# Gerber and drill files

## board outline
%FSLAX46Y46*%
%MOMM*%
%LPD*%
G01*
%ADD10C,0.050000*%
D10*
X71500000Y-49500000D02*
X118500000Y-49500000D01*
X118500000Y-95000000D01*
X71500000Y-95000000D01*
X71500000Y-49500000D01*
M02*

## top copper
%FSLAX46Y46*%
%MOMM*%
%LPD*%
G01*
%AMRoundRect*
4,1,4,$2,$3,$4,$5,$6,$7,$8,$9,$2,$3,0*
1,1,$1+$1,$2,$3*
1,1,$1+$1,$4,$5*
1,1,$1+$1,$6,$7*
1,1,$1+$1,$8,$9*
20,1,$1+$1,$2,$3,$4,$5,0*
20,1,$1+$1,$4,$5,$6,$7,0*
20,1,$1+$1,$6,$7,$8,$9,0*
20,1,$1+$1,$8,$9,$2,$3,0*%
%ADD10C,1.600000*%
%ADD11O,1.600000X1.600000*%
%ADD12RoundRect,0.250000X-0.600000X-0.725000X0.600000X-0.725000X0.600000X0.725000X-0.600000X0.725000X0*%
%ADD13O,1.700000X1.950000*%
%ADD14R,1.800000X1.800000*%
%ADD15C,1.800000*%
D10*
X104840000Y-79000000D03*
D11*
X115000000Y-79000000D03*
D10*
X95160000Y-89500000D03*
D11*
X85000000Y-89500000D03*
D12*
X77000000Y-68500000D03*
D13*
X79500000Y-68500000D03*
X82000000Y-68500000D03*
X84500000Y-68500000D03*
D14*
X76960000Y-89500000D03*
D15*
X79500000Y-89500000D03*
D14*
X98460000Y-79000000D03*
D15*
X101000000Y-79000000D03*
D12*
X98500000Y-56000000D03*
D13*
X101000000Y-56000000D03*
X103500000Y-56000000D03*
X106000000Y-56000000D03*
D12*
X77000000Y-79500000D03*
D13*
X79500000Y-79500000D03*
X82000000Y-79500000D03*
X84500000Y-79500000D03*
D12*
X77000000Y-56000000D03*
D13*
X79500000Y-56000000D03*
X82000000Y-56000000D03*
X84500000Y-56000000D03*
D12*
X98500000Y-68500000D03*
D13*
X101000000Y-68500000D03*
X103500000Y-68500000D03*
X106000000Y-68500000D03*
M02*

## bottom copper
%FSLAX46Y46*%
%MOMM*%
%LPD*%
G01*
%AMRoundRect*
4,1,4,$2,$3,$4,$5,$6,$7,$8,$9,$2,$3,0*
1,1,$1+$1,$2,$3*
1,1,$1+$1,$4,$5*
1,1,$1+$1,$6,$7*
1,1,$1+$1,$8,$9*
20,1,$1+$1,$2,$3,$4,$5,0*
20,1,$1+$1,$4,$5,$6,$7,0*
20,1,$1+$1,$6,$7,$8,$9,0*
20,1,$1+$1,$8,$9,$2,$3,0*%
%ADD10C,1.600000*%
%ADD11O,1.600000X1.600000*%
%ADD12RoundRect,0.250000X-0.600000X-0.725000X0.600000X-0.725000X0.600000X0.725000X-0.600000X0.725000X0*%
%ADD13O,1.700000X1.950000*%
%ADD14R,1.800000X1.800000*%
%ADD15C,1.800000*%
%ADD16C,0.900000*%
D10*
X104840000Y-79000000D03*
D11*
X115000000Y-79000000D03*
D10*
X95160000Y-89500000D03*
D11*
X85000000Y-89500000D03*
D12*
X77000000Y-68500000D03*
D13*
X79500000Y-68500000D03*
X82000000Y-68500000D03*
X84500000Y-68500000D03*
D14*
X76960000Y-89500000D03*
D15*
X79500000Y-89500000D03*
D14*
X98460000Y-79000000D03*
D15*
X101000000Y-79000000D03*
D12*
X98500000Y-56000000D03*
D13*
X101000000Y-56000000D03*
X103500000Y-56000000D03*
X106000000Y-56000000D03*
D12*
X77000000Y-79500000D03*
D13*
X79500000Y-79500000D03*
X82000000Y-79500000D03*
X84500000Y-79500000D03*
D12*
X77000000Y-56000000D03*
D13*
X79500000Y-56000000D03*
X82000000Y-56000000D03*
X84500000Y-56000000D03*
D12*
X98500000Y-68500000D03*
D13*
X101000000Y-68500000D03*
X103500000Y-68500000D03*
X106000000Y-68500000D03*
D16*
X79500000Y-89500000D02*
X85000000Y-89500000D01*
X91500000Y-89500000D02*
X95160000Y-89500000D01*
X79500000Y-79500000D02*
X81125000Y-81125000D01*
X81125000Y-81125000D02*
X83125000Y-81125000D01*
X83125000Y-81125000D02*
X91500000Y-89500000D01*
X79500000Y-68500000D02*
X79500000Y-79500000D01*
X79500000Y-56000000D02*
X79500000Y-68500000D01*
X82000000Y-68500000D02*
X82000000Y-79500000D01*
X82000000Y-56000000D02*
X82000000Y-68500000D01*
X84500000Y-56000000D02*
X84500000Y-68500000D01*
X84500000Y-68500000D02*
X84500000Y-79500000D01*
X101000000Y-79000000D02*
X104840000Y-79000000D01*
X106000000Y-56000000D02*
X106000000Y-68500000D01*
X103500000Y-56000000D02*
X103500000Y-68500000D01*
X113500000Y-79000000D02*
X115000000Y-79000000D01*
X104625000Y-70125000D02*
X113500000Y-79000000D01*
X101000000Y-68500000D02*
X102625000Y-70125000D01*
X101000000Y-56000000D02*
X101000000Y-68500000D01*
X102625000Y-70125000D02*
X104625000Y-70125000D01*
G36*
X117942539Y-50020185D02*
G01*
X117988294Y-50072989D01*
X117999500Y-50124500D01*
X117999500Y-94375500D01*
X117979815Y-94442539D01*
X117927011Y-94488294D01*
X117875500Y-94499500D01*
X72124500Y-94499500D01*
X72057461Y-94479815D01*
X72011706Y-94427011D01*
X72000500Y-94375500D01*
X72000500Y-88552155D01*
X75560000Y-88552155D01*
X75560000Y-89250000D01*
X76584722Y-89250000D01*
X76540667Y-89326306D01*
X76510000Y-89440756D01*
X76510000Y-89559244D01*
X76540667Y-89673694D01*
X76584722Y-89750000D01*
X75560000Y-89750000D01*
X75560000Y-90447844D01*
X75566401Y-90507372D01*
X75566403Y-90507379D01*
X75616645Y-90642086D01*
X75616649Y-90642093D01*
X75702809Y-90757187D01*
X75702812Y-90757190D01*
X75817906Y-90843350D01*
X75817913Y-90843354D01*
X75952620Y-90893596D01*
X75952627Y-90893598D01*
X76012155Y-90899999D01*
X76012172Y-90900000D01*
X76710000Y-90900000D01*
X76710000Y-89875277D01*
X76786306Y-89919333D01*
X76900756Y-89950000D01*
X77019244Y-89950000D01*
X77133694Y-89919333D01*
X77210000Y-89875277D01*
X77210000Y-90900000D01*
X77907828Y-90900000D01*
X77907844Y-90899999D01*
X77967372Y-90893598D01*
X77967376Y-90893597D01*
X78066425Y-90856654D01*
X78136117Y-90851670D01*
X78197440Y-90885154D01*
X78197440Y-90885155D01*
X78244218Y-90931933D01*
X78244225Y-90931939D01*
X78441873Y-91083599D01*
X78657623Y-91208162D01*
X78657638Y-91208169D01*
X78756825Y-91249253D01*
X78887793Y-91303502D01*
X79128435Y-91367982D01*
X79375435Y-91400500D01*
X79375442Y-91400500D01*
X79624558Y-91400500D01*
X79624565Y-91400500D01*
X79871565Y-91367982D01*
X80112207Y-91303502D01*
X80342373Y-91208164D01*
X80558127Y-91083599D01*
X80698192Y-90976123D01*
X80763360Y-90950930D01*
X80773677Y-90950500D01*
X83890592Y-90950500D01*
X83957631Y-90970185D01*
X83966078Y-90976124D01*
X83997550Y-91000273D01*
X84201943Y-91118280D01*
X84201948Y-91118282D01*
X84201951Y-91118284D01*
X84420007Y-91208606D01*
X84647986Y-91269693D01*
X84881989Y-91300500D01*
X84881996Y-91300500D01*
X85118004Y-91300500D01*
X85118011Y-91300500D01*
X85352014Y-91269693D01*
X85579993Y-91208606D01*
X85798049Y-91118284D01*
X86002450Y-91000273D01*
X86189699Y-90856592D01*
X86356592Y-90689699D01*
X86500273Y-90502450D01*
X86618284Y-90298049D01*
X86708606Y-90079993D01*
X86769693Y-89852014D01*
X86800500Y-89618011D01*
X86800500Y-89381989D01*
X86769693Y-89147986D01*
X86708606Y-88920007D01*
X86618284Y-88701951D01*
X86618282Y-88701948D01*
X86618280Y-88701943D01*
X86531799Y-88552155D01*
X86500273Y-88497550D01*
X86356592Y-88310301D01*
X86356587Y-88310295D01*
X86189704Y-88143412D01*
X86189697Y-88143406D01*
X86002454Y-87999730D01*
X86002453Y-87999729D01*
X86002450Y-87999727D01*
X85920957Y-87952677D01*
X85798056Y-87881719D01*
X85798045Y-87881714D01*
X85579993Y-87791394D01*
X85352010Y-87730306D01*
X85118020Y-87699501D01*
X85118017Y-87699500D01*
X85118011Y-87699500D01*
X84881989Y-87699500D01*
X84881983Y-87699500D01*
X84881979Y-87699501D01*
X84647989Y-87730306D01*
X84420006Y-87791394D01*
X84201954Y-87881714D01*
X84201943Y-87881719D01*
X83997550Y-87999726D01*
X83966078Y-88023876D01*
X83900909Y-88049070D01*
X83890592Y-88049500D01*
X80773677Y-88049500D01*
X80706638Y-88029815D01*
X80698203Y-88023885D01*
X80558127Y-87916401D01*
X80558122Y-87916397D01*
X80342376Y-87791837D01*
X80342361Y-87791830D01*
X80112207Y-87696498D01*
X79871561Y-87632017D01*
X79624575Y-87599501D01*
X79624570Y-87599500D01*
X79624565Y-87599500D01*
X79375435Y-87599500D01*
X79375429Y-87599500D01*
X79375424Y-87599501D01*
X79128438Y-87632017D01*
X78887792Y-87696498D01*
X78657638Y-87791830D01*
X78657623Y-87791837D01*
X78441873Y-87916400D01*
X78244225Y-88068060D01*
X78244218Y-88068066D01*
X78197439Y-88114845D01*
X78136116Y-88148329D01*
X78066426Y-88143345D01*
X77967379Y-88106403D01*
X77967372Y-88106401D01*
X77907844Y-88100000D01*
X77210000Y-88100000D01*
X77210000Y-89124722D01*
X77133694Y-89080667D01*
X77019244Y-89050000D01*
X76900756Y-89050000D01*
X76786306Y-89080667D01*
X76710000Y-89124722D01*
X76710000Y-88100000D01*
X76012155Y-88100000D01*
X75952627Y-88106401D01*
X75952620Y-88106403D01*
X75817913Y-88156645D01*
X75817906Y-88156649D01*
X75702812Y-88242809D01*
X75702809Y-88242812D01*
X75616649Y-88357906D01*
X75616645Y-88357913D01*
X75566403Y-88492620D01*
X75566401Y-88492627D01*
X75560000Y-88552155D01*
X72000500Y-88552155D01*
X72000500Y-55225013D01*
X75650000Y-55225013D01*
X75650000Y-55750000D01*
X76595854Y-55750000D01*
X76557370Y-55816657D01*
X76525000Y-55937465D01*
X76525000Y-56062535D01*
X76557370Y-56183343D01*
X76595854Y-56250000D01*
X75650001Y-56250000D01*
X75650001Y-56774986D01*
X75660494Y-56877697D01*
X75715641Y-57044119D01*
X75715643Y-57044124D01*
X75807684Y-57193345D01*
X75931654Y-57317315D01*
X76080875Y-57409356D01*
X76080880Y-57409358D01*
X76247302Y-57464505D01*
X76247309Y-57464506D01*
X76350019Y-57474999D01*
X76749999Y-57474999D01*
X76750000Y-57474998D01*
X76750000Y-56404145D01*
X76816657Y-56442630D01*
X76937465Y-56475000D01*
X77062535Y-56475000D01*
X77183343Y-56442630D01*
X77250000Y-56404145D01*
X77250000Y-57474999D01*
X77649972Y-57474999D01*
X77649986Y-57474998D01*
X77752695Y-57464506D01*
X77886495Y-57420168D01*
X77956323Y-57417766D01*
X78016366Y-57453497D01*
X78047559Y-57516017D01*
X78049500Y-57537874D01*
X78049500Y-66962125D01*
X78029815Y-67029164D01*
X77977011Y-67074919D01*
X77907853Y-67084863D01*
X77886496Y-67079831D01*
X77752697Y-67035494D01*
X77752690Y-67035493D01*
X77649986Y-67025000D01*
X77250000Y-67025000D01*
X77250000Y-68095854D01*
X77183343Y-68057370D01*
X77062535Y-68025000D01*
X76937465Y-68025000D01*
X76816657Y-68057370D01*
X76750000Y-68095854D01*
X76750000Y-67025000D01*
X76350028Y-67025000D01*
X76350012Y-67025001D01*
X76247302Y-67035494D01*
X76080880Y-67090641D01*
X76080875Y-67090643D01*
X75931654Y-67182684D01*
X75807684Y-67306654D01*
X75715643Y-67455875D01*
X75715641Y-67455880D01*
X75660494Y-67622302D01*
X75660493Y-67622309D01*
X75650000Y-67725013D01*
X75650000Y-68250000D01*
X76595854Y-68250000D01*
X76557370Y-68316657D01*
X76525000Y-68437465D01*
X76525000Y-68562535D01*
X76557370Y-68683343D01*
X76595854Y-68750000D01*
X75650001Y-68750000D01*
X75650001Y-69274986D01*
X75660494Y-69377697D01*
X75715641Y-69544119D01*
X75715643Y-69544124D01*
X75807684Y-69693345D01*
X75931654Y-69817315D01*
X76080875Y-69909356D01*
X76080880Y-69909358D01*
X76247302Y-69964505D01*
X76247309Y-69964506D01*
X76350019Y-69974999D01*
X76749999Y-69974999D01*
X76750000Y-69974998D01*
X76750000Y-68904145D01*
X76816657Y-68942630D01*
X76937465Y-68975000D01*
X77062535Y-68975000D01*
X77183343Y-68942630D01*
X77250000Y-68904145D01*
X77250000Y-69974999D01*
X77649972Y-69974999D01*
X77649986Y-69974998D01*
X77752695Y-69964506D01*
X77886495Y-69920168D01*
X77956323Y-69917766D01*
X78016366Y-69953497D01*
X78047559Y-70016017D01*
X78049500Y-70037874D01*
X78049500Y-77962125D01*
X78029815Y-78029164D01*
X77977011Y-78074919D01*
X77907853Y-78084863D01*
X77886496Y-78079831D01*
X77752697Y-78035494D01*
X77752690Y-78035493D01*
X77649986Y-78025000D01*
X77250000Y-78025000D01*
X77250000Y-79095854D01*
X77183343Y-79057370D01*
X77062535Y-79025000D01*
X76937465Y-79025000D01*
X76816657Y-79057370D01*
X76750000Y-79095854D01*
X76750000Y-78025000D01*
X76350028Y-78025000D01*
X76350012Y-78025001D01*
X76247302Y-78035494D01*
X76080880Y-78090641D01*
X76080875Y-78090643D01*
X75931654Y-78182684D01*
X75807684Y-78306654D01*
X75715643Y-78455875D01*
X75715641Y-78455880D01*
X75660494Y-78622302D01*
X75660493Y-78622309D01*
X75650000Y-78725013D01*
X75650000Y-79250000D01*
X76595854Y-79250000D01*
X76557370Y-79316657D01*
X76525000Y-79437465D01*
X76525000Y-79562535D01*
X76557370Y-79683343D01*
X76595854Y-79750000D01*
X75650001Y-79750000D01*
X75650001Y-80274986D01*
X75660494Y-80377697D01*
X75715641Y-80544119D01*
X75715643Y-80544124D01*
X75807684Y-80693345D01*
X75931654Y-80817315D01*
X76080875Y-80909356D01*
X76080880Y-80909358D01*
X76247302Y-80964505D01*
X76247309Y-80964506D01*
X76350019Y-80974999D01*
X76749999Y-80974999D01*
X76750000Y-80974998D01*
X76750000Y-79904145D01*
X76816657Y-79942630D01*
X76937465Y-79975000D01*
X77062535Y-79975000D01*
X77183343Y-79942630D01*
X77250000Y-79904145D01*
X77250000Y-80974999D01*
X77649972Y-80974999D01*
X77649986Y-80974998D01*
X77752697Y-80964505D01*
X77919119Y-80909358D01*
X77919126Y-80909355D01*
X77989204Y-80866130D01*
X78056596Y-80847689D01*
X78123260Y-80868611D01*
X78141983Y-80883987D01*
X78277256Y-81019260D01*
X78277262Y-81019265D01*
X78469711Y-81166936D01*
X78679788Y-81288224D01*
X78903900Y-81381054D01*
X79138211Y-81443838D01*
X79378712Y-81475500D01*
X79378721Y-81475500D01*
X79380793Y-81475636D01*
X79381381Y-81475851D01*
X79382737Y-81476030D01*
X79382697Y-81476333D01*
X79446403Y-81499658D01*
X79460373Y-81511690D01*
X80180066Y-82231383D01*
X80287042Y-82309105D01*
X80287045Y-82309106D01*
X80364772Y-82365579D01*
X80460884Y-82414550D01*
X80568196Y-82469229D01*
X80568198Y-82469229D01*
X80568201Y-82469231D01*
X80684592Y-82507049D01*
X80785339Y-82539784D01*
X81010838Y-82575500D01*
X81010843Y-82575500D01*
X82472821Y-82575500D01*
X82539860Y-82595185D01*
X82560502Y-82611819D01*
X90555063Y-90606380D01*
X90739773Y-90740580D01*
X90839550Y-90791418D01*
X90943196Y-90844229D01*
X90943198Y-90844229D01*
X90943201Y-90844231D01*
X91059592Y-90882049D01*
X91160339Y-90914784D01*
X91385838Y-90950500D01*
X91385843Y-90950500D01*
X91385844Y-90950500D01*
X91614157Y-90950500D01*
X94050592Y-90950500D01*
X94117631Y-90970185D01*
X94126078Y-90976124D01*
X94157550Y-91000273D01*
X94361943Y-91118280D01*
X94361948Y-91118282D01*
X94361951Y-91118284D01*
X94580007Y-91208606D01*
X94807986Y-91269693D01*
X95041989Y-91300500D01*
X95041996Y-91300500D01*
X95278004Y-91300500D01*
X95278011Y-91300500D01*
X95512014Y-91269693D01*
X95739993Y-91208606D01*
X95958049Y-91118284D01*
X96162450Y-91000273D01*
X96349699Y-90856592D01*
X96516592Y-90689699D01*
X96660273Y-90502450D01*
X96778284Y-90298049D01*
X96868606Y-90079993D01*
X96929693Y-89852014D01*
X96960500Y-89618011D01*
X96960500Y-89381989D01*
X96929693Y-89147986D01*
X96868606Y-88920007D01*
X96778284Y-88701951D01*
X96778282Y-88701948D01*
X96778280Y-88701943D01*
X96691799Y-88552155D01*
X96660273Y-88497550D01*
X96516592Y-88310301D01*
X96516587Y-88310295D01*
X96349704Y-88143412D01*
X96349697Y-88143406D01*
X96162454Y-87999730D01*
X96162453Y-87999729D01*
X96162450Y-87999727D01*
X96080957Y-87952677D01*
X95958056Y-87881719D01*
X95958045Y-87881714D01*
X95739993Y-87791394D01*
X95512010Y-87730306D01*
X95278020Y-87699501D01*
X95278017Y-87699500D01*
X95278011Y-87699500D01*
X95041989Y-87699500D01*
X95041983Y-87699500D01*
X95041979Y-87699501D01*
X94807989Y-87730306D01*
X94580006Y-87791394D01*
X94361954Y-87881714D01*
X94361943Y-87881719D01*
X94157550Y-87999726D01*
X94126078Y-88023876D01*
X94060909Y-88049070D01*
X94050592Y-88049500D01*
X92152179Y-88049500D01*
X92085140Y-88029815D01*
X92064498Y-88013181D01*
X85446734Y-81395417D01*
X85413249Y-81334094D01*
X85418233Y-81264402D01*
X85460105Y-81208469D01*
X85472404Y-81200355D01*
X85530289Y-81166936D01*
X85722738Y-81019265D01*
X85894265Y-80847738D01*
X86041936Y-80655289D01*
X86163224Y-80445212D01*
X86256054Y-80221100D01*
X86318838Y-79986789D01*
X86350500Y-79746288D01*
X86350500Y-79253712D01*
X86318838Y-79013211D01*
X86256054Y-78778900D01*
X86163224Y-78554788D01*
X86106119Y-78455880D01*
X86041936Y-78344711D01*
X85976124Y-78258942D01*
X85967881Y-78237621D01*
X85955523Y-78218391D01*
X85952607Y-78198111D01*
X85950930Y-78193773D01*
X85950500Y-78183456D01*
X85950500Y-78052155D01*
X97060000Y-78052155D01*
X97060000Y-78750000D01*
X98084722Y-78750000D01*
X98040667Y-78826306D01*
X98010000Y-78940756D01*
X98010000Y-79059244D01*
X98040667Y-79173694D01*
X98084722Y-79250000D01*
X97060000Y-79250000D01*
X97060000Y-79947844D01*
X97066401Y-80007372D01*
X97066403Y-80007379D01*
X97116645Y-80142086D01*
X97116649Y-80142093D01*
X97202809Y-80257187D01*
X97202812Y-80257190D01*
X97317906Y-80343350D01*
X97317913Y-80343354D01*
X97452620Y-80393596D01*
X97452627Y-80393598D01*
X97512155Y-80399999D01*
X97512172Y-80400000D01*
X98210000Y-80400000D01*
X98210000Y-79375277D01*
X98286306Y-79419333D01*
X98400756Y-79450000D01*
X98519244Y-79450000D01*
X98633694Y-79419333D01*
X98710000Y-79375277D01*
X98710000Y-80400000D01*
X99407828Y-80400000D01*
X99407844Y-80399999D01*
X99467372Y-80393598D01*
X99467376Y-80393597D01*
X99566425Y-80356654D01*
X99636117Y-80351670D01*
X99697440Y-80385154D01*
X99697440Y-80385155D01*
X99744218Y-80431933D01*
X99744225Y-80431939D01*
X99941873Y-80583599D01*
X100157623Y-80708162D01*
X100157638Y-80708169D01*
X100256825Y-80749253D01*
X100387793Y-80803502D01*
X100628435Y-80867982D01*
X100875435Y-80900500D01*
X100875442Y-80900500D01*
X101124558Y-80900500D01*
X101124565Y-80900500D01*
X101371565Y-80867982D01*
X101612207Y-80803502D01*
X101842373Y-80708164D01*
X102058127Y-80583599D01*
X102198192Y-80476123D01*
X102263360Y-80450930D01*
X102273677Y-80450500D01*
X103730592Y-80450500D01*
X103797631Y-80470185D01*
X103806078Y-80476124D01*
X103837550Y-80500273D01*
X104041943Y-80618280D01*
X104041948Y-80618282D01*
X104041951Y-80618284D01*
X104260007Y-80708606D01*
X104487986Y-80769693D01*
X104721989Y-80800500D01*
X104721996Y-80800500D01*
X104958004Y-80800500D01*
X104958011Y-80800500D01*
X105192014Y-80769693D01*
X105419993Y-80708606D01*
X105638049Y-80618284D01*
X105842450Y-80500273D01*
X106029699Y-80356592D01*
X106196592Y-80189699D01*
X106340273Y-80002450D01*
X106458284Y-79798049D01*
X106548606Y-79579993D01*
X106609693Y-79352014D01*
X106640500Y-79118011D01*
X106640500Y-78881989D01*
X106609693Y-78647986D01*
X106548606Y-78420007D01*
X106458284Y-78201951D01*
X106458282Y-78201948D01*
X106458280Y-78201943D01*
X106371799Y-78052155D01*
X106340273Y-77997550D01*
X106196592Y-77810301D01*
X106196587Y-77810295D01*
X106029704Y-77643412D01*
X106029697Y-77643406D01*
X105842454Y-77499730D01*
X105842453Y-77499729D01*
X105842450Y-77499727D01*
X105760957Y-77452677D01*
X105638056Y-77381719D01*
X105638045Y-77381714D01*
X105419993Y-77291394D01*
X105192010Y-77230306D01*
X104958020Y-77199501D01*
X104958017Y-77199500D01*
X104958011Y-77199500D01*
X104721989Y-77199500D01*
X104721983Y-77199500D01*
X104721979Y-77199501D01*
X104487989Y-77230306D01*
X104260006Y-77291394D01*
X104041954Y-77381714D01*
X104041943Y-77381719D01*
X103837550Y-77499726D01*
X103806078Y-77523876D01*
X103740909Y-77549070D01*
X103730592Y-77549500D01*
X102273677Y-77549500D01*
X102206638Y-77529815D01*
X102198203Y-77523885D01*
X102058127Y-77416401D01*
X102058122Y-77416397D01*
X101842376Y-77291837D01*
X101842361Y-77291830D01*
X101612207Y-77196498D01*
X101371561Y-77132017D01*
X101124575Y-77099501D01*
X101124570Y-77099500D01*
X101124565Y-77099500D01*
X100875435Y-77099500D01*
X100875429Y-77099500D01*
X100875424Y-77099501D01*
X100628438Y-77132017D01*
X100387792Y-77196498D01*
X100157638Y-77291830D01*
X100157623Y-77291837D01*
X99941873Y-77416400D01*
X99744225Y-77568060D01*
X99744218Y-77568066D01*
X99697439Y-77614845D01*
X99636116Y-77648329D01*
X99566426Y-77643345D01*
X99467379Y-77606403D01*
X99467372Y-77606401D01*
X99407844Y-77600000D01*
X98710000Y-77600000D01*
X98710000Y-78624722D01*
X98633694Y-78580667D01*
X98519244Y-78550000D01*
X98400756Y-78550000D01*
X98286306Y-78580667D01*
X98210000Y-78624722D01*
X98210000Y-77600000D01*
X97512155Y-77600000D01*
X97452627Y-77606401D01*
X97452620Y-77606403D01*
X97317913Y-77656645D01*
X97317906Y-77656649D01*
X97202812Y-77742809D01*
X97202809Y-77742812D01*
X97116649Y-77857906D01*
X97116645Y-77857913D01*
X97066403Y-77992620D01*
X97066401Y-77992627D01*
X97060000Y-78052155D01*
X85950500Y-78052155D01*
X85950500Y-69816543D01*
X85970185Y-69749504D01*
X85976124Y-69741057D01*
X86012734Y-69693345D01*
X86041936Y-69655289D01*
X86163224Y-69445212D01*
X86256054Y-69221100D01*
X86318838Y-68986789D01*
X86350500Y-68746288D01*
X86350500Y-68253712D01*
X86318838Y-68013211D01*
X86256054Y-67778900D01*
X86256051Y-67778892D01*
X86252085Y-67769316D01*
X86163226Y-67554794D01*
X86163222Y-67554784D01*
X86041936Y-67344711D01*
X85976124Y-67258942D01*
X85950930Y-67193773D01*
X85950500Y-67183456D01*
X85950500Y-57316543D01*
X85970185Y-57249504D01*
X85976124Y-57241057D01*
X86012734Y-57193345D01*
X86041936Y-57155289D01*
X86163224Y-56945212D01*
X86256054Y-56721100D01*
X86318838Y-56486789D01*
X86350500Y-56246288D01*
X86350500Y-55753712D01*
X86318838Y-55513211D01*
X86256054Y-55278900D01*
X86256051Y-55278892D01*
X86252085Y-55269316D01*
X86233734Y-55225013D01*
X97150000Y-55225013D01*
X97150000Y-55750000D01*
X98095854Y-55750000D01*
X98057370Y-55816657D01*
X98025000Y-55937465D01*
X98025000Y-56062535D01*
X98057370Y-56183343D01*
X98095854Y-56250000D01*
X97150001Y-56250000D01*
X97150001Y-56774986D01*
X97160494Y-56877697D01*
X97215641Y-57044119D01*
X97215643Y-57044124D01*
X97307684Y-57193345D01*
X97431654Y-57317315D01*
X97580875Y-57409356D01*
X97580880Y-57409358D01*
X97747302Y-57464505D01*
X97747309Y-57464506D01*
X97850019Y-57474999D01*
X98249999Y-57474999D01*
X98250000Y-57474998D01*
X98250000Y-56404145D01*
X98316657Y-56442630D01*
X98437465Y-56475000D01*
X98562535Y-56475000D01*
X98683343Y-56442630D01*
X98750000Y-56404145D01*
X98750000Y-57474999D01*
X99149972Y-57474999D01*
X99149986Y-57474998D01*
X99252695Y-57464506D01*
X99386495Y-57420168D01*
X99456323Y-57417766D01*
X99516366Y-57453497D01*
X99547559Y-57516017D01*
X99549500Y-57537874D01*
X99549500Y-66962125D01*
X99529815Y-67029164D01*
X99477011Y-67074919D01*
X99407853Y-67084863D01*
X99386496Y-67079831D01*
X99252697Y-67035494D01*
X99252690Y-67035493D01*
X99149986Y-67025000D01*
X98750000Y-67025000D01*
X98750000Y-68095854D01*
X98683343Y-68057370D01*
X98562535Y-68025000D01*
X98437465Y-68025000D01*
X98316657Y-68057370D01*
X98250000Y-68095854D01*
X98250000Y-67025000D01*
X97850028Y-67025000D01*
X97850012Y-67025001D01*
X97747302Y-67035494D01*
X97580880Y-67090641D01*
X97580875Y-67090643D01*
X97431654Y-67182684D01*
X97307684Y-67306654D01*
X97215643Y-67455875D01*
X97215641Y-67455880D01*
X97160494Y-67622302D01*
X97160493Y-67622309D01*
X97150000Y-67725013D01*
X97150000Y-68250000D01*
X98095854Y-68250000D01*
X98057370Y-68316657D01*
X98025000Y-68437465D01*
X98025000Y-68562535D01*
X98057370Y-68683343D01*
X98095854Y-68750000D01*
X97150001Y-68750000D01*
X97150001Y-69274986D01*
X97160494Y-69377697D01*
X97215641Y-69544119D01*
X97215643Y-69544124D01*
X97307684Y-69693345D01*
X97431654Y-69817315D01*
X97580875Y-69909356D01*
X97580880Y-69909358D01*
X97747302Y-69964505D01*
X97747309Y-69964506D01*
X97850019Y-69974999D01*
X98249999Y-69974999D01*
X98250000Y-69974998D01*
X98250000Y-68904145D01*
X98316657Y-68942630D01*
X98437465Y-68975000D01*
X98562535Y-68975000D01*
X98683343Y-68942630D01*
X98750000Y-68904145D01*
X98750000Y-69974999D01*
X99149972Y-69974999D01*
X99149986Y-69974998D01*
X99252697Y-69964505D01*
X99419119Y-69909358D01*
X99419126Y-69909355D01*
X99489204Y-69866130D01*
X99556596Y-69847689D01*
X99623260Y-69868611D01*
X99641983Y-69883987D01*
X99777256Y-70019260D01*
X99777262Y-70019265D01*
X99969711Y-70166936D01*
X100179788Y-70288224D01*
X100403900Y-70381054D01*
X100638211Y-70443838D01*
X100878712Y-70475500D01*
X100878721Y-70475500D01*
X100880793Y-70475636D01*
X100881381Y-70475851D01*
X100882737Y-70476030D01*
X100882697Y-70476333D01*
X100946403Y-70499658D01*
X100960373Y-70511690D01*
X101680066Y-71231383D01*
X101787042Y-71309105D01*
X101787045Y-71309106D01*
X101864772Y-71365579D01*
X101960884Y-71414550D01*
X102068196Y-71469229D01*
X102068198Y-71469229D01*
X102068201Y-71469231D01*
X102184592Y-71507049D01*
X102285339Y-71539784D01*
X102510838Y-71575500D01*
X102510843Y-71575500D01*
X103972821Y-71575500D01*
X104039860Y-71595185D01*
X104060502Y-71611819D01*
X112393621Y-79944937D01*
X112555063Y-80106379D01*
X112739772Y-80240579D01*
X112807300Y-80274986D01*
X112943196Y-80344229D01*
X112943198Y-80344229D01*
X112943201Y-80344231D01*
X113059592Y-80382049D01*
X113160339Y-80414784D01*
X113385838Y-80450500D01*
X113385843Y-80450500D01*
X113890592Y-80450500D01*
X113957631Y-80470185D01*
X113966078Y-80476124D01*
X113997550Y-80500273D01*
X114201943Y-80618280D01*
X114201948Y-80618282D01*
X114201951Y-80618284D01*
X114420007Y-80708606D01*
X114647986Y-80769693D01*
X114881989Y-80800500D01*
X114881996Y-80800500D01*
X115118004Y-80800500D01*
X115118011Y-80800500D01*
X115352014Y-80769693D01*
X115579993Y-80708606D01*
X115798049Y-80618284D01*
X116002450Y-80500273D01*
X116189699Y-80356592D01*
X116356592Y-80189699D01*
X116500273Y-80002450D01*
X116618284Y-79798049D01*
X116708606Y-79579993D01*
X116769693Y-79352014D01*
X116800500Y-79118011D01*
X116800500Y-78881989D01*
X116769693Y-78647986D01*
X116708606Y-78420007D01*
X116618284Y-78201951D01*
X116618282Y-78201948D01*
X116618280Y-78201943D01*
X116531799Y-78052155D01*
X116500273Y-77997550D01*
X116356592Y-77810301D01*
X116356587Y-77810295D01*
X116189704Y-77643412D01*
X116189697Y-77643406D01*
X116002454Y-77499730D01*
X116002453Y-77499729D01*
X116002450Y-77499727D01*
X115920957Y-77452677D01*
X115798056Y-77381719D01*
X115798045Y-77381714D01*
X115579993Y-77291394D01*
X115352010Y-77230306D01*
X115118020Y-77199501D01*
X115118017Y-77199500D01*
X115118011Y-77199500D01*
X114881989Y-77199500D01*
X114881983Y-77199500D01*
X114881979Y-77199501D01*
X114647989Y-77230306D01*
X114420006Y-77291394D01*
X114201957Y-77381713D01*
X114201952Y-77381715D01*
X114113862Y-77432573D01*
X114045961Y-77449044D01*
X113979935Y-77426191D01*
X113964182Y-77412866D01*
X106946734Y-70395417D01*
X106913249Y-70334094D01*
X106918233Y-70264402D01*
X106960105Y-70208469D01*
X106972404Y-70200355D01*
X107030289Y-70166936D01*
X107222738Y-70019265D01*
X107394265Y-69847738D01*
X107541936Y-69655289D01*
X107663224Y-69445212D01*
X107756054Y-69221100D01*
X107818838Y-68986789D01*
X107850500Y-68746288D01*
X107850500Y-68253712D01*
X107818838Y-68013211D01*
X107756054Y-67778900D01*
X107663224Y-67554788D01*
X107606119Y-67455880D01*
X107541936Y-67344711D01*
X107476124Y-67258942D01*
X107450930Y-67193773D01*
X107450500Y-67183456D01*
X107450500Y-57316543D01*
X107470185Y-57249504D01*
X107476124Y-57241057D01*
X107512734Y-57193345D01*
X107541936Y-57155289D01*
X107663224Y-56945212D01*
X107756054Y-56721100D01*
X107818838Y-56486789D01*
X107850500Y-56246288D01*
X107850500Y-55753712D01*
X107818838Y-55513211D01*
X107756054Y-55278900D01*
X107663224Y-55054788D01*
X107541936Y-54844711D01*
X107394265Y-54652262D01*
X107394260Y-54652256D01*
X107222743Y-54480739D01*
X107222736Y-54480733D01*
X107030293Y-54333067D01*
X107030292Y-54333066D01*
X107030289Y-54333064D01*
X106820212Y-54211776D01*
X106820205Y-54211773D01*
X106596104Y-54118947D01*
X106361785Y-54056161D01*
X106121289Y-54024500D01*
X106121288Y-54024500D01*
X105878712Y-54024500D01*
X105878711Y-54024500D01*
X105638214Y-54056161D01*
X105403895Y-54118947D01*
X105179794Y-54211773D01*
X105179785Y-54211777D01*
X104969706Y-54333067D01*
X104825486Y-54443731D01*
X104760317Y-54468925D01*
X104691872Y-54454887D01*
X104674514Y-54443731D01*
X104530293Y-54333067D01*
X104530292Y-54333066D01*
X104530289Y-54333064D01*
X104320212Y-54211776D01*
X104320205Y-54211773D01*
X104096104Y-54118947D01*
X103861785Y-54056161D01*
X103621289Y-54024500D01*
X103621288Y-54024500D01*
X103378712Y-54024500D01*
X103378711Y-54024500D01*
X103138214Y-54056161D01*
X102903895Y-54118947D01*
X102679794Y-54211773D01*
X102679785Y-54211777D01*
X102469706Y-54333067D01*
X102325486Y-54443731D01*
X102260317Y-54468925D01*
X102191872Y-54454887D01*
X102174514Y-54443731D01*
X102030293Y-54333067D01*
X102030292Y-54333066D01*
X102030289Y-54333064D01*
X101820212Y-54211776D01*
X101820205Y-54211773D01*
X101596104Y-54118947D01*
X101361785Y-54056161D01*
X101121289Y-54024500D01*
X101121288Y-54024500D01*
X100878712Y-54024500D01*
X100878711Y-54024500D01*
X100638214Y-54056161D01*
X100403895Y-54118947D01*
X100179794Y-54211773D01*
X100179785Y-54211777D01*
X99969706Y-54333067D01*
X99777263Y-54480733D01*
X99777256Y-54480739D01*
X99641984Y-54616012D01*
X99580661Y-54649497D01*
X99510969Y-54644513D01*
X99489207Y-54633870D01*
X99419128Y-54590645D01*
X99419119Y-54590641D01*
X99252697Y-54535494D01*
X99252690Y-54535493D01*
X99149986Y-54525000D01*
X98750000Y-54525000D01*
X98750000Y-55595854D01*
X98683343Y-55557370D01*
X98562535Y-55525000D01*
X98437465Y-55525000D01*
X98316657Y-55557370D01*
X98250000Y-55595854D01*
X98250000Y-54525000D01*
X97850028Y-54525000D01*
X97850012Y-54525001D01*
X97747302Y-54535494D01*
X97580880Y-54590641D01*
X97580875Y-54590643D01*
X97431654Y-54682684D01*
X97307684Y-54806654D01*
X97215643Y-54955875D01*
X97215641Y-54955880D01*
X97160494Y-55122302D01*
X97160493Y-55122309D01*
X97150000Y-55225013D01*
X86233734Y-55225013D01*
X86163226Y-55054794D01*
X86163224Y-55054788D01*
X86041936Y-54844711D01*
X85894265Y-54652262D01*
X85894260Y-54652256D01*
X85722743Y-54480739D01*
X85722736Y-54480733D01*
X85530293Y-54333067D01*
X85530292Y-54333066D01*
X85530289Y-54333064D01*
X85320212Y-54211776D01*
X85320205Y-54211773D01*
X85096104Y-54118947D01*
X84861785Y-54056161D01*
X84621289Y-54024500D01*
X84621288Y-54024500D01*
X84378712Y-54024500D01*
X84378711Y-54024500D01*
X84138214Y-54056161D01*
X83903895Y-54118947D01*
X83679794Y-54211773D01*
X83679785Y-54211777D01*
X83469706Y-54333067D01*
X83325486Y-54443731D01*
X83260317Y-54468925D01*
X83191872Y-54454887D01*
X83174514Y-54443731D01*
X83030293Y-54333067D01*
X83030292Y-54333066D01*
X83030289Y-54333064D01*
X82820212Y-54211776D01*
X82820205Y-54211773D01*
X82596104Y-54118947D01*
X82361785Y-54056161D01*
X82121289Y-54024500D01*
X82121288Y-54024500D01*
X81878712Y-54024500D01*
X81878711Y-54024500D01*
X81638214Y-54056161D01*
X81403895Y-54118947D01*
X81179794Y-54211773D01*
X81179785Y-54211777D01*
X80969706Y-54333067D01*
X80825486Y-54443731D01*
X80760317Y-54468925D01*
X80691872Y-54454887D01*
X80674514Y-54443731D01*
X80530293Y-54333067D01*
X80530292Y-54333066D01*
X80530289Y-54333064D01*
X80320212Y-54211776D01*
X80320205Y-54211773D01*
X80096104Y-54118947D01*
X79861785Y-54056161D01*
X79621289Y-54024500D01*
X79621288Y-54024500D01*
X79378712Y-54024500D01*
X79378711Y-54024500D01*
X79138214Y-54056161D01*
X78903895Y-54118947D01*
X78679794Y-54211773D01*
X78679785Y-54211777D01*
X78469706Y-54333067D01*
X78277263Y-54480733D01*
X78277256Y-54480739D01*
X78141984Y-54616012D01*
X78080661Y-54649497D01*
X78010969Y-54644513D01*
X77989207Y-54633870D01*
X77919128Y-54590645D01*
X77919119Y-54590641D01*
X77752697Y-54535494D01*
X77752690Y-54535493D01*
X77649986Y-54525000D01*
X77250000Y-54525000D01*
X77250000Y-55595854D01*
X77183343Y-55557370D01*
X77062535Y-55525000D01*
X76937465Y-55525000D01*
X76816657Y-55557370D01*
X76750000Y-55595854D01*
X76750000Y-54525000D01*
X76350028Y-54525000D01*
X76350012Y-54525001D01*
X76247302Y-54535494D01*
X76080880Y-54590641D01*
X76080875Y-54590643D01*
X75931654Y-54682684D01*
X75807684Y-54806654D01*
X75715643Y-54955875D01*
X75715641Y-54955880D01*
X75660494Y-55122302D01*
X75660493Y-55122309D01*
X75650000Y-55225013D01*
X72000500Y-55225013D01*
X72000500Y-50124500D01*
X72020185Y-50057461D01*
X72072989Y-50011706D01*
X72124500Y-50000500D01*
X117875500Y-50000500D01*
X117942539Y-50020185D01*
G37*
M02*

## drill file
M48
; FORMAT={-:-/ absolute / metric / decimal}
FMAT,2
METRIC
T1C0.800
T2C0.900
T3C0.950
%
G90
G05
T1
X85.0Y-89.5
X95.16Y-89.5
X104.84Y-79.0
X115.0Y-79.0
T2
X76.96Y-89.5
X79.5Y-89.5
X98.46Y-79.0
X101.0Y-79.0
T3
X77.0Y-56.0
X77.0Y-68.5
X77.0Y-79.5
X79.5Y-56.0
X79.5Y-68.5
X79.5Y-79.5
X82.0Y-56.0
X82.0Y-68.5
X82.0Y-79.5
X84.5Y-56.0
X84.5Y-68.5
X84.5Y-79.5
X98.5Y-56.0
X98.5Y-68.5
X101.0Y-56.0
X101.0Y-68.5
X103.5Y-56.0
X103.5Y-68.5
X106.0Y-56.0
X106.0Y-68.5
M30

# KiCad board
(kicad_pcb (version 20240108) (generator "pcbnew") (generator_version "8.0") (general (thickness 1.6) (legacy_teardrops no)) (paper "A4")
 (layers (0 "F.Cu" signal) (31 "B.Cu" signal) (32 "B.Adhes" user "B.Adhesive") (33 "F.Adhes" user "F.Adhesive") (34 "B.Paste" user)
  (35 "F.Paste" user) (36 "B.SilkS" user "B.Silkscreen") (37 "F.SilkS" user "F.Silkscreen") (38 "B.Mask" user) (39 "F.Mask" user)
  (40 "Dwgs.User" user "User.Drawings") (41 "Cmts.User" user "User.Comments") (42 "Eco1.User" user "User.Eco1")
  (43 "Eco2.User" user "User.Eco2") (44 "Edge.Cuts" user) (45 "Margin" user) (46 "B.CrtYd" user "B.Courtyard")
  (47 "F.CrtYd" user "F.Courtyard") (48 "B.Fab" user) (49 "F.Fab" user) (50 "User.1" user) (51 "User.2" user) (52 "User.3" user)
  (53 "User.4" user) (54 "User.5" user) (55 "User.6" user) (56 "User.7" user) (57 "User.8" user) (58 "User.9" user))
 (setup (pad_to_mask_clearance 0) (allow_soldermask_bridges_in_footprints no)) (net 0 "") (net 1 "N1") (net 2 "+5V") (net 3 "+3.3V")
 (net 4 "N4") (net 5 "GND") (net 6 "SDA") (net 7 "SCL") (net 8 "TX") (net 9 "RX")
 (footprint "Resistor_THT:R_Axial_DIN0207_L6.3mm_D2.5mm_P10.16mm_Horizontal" (layer "F.Cu") (at 104.84 79)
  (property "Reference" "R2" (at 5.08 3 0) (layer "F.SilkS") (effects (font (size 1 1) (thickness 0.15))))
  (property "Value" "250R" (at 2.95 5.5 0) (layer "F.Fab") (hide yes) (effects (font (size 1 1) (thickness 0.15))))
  (pad "1" thru_hole circle (at 0 0) (size 1.6 1.6) (drill 0.8) (layers "*.Cu" "*.Mask") (remove_unused_layers no) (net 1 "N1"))
  (pad "2" thru_hole oval (at 10.16 0) (size 1.6 1.6) (drill 0.8) (layers "*.Cu" "*.Mask") (remove_unused_layers no) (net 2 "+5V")))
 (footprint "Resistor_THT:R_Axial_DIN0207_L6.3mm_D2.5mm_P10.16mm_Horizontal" (layer "F.Cu") (at 95.16 89.5 180)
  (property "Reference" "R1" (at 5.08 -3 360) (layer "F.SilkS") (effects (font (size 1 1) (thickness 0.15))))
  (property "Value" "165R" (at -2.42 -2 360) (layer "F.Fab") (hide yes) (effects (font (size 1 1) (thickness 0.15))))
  (pad "1" thru_hole circle (at 0 0 180) (size 1.6 1.6) (drill 0.8) (layers "*.Cu" "*.Mask") (remove_unused_layers no) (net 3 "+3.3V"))
  (pad "2" thru_hole oval (at 10.16 0 180) (size 1.6 1.6) (drill 0.8) (layers "*.Cu" "*.Mask") (remove_unused_layers no) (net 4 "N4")))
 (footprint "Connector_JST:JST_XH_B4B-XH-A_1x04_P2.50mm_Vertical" (layer "F.Cu") (at 77 68.5)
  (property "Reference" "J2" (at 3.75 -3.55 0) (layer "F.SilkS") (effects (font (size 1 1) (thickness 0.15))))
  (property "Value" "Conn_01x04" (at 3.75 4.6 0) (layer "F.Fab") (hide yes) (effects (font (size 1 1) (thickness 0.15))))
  (pad "1" thru_hole roundrect (at 0 0) (size 1.7 1.95) (drill 0.95) (layers "*.Cu" "*.Mask") (remove_unused_layers no)
   (roundrect_rratio 0.147059) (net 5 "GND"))
  (pad "2" thru_hole oval (at 2.5 0) (size 1.7 1.95) (drill 0.95) (layers "*.Cu" "*.Mask") (remove_unused_layers no) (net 3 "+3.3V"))
  (pad "3" thru_hole oval (at 5 0) (size 1.7 1.95) (drill 0.95) (layers "*.Cu" "*.Mask") (remove_unused_layers no) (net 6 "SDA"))
  (pad "4" thru_hole oval (at 7.5 0) (size 1.7 1.95) (drill 0.95) (layers "*.Cu" "*.Mask") (remove_unused_layers no) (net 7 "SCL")))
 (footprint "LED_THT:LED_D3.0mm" (layer "F.Cu") (at 76.96 89.5)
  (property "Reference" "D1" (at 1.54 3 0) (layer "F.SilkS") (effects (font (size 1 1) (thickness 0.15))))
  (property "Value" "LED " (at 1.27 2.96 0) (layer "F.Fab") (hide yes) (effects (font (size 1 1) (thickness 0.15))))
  (pad "1" thru_hole rect (at 0 0) (size 1.8 1.8) (drill 0.9) (layers "*.Cu" "*.Mask") (remove_unused_layers no) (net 5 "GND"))
  (pad "2" thru_hole circle (at 2.54 0) (size 1.8 1.8) (drill 0.9) (layers "*.Cu" "*.Mask") (remove_unused_layers no) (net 4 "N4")))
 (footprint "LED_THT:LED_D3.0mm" (layer "F.Cu") (at 98.46 79)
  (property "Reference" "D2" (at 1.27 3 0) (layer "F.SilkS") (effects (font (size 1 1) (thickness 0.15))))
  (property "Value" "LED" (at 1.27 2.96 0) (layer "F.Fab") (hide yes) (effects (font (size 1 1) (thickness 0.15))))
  (pad "1" thru_hole rect (at 0 0) (size 1.8 1.8) (drill 0.9) (layers "*.Cu" "*.Mask") (remove_unused_layers no) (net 5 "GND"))
  (pad "2" thru_hole circle (at 2.54 0) (size 1.8 1.8) (drill 0.9) (layers "*.Cu" "*.Mask") (remove_unused_layers no) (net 1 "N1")))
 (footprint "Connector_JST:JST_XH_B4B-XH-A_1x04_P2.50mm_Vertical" (layer "F.Cu") (at 98.5 56)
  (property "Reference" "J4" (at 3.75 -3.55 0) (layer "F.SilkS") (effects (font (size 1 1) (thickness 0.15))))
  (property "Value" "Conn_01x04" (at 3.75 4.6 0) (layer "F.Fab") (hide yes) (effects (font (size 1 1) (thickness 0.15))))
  (pad "1" thru_hole roundrect (at 0 0) (size 1.7 1.95) (drill 0.95) (layers "*.Cu" "*.Mask") (remove_unused_layers no)
   (roundrect_rratio 0.147059) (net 5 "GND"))
  (pad "2" thru_hole oval (at 2.5 0) (size 1.7 1.95) (drill 0.95) (layers "*.Cu" "*.Mask") (remove_unused_layers no) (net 2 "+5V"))
  (pad "3" thru_hole oval (at 5 0) (size 1.7 1.95) (drill 0.95) (layers "*.Cu" "*.Mask") (remove_unused_layers no) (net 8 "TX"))
  (pad "4" thru_hole oval (at 7.5 0) (size 1.7 1.95) (drill 0.95) (layers "*.Cu" "*.Mask") (remove_unused_layers no) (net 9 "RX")))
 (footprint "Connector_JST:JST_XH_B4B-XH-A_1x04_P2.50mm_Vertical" (layer "F.Cu") (at 77 79.5)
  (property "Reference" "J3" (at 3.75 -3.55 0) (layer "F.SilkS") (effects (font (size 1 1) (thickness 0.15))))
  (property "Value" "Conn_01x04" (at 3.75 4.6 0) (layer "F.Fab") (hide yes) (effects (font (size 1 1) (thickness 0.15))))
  (pad "1" thru_hole roundrect (at 0 0) (size 1.7 1.95) (drill 0.95) (layers "*.Cu" "*.Mask") (remove_unused_layers no)
   (roundrect_rratio 0.147059) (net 5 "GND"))
  (pad "2" thru_hole oval (at 2.5 0) (size 1.7 1.95) (drill 0.95) (layers "*.Cu" "*.Mask") (remove_unused_layers no) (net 3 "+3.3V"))
  (pad "3" thru_hole oval (at 5 0) (size 1.7 1.95) (drill 0.95) (layers "*.Cu" "*.Mask") (remove_unused_layers no) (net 6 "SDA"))
  (pad "4" thru_hole oval (at 7.5 0) (size 1.7 1.95) (drill 0.95) (layers "*.Cu" "*.Mask") (remove_unused_layers no) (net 7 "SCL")))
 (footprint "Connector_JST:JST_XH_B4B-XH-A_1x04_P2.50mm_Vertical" (layer "F.Cu") (at 77 56)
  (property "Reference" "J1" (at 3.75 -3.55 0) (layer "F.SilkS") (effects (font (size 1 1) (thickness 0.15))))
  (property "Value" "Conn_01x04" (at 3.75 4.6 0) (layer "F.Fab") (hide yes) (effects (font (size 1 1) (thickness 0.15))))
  (pad "1" thru_hole roundrect (at 0 0) (size 1.7 1.95) (drill 0.95) (layers "*.Cu" "*.Mask") (remove_unused_layers no)
   (roundrect_rratio 0.147059) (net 5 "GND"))
  (pad "2" thru_hole oval (at 2.5 0) (size 1.7 1.95) (drill 0.95) (layers "*.Cu" "*.Mask") (remove_unused_layers no) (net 3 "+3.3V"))
  (pad "3" thru_hole oval (at 5 0) (size 1.7 1.95) (drill 0.95) (layers "*.Cu" "*.Mask") (remove_unused_layers no) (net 6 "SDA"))
  (pad "4" thru_hole oval (at 7.5 0) (size 1.7 1.95) (drill 0.95) (layers "*.Cu" "*.Mask") (remove_unused_layers no) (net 7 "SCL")))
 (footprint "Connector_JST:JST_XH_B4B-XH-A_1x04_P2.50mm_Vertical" (layer "F.Cu") (at 98.5 68.5)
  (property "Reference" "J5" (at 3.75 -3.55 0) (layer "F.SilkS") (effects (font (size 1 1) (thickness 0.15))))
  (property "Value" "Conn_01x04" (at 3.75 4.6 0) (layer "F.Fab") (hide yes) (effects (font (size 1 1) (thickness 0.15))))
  (pad "1" thru_hole roundrect (at 0 0) (size 1.7 1.95) (drill 0.95) (layers "*.Cu" "*.Mask") (remove_unused_layers no)
   (roundrect_rratio 0.147059) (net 5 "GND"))
  (pad "2" thru_hole oval (at 2.5 0) (size 1.7 1.95) (drill 0.95) (layers "*.Cu" "*.Mask") (remove_unused_layers no) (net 2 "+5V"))
  (pad "3" thru_hole oval (at 5 0) (size 1.7 1.95) (drill 0.95) (layers "*.Cu" "*.Mask") (remove_unused_layers no) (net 8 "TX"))
  (pad "4" thru_hole oval (at 7.5 0) (size 1.7 1.95) (drill 0.95) (layers "*.Cu" "*.Mask") (remove_unused_layers no) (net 9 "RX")))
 (gr_rect (start 71.5 49.5) (end 118.5 95) (stroke (width 0.05) (type default)) (fill none) (layer "Edge.Cuts"))
 (segment (start 79.5 89.5) (end 85 89.5) (width 0.9) (layer "B.Cu") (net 4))
 (segment (start 91.5 89.5) (end 95.16 89.5) (width 0.9) (layer "B.Cu") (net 3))
 (segment (start 79.5 79.5) (end 81.125 81.125) (width 0.9) (layer "B.Cu") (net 3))
 (segment (start 81.125 81.125) (end 83.125 81.125) (width 0.9) (layer "B.Cu") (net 3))
 (segment (start 83.125 81.125) (end 91.5 89.5) (width 0.9) (layer "B.Cu") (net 3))
 (segment (start 79.5 68.5) (end 79.5 79.5) (width 0.9) (layer "B.Cu") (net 3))
 (segment (start 79.5 56) (end 79.5 68.5) (width 0.9) (layer "B.Cu") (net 3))
 (segment (start 82 68.5) (end 82 79.5) (width 0.9) (layer "B.Cu") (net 6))
 (segment (start 82 56) (end 82 68.5) (width 0.9) (layer "B.Cu") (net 6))
 (segment (start 84.5 56) (end 84.5 68.5) (width 0.9) (layer "B.Cu") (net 7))
 (segment (start 84.5 68.5) (end 84.5 79.5) (width 0.9) (layer "B.Cu") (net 7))
 (segment (start 101 79) (end 104.84 79) (width 0.9) (layer "B.Cu") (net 1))
 (segment (start 106 56) (end 106 68.5) (width 0.9) (layer "B.Cu") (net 9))
 (segment (start 103.5 56) (end 103.5 68.5) (width 0.9) (layer "B.Cu") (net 8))
 (segment (start 113.5 79) (end 115 79) (width 0.9) (layer "B.Cu") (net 2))
 (segment (start 104.625 70.125) (end 113.5 79) (width 0.9) (layer "B.Cu") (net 2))
 (segment (start 101 68.5) (end 102.625 70.125) (width 0.9) (layer "B.Cu") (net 2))
 (segment (start 101 56) (end 101 68.5) (width 0.9) (layer "B.Cu") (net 2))
 (segment (start 102.625 70.125) (end 104.625 70.125) (width 0.9) (layer "B.Cu") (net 2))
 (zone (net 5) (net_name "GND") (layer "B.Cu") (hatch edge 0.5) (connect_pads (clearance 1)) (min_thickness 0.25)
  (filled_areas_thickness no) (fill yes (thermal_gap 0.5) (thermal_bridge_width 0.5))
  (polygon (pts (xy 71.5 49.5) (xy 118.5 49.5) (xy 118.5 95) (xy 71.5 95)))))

